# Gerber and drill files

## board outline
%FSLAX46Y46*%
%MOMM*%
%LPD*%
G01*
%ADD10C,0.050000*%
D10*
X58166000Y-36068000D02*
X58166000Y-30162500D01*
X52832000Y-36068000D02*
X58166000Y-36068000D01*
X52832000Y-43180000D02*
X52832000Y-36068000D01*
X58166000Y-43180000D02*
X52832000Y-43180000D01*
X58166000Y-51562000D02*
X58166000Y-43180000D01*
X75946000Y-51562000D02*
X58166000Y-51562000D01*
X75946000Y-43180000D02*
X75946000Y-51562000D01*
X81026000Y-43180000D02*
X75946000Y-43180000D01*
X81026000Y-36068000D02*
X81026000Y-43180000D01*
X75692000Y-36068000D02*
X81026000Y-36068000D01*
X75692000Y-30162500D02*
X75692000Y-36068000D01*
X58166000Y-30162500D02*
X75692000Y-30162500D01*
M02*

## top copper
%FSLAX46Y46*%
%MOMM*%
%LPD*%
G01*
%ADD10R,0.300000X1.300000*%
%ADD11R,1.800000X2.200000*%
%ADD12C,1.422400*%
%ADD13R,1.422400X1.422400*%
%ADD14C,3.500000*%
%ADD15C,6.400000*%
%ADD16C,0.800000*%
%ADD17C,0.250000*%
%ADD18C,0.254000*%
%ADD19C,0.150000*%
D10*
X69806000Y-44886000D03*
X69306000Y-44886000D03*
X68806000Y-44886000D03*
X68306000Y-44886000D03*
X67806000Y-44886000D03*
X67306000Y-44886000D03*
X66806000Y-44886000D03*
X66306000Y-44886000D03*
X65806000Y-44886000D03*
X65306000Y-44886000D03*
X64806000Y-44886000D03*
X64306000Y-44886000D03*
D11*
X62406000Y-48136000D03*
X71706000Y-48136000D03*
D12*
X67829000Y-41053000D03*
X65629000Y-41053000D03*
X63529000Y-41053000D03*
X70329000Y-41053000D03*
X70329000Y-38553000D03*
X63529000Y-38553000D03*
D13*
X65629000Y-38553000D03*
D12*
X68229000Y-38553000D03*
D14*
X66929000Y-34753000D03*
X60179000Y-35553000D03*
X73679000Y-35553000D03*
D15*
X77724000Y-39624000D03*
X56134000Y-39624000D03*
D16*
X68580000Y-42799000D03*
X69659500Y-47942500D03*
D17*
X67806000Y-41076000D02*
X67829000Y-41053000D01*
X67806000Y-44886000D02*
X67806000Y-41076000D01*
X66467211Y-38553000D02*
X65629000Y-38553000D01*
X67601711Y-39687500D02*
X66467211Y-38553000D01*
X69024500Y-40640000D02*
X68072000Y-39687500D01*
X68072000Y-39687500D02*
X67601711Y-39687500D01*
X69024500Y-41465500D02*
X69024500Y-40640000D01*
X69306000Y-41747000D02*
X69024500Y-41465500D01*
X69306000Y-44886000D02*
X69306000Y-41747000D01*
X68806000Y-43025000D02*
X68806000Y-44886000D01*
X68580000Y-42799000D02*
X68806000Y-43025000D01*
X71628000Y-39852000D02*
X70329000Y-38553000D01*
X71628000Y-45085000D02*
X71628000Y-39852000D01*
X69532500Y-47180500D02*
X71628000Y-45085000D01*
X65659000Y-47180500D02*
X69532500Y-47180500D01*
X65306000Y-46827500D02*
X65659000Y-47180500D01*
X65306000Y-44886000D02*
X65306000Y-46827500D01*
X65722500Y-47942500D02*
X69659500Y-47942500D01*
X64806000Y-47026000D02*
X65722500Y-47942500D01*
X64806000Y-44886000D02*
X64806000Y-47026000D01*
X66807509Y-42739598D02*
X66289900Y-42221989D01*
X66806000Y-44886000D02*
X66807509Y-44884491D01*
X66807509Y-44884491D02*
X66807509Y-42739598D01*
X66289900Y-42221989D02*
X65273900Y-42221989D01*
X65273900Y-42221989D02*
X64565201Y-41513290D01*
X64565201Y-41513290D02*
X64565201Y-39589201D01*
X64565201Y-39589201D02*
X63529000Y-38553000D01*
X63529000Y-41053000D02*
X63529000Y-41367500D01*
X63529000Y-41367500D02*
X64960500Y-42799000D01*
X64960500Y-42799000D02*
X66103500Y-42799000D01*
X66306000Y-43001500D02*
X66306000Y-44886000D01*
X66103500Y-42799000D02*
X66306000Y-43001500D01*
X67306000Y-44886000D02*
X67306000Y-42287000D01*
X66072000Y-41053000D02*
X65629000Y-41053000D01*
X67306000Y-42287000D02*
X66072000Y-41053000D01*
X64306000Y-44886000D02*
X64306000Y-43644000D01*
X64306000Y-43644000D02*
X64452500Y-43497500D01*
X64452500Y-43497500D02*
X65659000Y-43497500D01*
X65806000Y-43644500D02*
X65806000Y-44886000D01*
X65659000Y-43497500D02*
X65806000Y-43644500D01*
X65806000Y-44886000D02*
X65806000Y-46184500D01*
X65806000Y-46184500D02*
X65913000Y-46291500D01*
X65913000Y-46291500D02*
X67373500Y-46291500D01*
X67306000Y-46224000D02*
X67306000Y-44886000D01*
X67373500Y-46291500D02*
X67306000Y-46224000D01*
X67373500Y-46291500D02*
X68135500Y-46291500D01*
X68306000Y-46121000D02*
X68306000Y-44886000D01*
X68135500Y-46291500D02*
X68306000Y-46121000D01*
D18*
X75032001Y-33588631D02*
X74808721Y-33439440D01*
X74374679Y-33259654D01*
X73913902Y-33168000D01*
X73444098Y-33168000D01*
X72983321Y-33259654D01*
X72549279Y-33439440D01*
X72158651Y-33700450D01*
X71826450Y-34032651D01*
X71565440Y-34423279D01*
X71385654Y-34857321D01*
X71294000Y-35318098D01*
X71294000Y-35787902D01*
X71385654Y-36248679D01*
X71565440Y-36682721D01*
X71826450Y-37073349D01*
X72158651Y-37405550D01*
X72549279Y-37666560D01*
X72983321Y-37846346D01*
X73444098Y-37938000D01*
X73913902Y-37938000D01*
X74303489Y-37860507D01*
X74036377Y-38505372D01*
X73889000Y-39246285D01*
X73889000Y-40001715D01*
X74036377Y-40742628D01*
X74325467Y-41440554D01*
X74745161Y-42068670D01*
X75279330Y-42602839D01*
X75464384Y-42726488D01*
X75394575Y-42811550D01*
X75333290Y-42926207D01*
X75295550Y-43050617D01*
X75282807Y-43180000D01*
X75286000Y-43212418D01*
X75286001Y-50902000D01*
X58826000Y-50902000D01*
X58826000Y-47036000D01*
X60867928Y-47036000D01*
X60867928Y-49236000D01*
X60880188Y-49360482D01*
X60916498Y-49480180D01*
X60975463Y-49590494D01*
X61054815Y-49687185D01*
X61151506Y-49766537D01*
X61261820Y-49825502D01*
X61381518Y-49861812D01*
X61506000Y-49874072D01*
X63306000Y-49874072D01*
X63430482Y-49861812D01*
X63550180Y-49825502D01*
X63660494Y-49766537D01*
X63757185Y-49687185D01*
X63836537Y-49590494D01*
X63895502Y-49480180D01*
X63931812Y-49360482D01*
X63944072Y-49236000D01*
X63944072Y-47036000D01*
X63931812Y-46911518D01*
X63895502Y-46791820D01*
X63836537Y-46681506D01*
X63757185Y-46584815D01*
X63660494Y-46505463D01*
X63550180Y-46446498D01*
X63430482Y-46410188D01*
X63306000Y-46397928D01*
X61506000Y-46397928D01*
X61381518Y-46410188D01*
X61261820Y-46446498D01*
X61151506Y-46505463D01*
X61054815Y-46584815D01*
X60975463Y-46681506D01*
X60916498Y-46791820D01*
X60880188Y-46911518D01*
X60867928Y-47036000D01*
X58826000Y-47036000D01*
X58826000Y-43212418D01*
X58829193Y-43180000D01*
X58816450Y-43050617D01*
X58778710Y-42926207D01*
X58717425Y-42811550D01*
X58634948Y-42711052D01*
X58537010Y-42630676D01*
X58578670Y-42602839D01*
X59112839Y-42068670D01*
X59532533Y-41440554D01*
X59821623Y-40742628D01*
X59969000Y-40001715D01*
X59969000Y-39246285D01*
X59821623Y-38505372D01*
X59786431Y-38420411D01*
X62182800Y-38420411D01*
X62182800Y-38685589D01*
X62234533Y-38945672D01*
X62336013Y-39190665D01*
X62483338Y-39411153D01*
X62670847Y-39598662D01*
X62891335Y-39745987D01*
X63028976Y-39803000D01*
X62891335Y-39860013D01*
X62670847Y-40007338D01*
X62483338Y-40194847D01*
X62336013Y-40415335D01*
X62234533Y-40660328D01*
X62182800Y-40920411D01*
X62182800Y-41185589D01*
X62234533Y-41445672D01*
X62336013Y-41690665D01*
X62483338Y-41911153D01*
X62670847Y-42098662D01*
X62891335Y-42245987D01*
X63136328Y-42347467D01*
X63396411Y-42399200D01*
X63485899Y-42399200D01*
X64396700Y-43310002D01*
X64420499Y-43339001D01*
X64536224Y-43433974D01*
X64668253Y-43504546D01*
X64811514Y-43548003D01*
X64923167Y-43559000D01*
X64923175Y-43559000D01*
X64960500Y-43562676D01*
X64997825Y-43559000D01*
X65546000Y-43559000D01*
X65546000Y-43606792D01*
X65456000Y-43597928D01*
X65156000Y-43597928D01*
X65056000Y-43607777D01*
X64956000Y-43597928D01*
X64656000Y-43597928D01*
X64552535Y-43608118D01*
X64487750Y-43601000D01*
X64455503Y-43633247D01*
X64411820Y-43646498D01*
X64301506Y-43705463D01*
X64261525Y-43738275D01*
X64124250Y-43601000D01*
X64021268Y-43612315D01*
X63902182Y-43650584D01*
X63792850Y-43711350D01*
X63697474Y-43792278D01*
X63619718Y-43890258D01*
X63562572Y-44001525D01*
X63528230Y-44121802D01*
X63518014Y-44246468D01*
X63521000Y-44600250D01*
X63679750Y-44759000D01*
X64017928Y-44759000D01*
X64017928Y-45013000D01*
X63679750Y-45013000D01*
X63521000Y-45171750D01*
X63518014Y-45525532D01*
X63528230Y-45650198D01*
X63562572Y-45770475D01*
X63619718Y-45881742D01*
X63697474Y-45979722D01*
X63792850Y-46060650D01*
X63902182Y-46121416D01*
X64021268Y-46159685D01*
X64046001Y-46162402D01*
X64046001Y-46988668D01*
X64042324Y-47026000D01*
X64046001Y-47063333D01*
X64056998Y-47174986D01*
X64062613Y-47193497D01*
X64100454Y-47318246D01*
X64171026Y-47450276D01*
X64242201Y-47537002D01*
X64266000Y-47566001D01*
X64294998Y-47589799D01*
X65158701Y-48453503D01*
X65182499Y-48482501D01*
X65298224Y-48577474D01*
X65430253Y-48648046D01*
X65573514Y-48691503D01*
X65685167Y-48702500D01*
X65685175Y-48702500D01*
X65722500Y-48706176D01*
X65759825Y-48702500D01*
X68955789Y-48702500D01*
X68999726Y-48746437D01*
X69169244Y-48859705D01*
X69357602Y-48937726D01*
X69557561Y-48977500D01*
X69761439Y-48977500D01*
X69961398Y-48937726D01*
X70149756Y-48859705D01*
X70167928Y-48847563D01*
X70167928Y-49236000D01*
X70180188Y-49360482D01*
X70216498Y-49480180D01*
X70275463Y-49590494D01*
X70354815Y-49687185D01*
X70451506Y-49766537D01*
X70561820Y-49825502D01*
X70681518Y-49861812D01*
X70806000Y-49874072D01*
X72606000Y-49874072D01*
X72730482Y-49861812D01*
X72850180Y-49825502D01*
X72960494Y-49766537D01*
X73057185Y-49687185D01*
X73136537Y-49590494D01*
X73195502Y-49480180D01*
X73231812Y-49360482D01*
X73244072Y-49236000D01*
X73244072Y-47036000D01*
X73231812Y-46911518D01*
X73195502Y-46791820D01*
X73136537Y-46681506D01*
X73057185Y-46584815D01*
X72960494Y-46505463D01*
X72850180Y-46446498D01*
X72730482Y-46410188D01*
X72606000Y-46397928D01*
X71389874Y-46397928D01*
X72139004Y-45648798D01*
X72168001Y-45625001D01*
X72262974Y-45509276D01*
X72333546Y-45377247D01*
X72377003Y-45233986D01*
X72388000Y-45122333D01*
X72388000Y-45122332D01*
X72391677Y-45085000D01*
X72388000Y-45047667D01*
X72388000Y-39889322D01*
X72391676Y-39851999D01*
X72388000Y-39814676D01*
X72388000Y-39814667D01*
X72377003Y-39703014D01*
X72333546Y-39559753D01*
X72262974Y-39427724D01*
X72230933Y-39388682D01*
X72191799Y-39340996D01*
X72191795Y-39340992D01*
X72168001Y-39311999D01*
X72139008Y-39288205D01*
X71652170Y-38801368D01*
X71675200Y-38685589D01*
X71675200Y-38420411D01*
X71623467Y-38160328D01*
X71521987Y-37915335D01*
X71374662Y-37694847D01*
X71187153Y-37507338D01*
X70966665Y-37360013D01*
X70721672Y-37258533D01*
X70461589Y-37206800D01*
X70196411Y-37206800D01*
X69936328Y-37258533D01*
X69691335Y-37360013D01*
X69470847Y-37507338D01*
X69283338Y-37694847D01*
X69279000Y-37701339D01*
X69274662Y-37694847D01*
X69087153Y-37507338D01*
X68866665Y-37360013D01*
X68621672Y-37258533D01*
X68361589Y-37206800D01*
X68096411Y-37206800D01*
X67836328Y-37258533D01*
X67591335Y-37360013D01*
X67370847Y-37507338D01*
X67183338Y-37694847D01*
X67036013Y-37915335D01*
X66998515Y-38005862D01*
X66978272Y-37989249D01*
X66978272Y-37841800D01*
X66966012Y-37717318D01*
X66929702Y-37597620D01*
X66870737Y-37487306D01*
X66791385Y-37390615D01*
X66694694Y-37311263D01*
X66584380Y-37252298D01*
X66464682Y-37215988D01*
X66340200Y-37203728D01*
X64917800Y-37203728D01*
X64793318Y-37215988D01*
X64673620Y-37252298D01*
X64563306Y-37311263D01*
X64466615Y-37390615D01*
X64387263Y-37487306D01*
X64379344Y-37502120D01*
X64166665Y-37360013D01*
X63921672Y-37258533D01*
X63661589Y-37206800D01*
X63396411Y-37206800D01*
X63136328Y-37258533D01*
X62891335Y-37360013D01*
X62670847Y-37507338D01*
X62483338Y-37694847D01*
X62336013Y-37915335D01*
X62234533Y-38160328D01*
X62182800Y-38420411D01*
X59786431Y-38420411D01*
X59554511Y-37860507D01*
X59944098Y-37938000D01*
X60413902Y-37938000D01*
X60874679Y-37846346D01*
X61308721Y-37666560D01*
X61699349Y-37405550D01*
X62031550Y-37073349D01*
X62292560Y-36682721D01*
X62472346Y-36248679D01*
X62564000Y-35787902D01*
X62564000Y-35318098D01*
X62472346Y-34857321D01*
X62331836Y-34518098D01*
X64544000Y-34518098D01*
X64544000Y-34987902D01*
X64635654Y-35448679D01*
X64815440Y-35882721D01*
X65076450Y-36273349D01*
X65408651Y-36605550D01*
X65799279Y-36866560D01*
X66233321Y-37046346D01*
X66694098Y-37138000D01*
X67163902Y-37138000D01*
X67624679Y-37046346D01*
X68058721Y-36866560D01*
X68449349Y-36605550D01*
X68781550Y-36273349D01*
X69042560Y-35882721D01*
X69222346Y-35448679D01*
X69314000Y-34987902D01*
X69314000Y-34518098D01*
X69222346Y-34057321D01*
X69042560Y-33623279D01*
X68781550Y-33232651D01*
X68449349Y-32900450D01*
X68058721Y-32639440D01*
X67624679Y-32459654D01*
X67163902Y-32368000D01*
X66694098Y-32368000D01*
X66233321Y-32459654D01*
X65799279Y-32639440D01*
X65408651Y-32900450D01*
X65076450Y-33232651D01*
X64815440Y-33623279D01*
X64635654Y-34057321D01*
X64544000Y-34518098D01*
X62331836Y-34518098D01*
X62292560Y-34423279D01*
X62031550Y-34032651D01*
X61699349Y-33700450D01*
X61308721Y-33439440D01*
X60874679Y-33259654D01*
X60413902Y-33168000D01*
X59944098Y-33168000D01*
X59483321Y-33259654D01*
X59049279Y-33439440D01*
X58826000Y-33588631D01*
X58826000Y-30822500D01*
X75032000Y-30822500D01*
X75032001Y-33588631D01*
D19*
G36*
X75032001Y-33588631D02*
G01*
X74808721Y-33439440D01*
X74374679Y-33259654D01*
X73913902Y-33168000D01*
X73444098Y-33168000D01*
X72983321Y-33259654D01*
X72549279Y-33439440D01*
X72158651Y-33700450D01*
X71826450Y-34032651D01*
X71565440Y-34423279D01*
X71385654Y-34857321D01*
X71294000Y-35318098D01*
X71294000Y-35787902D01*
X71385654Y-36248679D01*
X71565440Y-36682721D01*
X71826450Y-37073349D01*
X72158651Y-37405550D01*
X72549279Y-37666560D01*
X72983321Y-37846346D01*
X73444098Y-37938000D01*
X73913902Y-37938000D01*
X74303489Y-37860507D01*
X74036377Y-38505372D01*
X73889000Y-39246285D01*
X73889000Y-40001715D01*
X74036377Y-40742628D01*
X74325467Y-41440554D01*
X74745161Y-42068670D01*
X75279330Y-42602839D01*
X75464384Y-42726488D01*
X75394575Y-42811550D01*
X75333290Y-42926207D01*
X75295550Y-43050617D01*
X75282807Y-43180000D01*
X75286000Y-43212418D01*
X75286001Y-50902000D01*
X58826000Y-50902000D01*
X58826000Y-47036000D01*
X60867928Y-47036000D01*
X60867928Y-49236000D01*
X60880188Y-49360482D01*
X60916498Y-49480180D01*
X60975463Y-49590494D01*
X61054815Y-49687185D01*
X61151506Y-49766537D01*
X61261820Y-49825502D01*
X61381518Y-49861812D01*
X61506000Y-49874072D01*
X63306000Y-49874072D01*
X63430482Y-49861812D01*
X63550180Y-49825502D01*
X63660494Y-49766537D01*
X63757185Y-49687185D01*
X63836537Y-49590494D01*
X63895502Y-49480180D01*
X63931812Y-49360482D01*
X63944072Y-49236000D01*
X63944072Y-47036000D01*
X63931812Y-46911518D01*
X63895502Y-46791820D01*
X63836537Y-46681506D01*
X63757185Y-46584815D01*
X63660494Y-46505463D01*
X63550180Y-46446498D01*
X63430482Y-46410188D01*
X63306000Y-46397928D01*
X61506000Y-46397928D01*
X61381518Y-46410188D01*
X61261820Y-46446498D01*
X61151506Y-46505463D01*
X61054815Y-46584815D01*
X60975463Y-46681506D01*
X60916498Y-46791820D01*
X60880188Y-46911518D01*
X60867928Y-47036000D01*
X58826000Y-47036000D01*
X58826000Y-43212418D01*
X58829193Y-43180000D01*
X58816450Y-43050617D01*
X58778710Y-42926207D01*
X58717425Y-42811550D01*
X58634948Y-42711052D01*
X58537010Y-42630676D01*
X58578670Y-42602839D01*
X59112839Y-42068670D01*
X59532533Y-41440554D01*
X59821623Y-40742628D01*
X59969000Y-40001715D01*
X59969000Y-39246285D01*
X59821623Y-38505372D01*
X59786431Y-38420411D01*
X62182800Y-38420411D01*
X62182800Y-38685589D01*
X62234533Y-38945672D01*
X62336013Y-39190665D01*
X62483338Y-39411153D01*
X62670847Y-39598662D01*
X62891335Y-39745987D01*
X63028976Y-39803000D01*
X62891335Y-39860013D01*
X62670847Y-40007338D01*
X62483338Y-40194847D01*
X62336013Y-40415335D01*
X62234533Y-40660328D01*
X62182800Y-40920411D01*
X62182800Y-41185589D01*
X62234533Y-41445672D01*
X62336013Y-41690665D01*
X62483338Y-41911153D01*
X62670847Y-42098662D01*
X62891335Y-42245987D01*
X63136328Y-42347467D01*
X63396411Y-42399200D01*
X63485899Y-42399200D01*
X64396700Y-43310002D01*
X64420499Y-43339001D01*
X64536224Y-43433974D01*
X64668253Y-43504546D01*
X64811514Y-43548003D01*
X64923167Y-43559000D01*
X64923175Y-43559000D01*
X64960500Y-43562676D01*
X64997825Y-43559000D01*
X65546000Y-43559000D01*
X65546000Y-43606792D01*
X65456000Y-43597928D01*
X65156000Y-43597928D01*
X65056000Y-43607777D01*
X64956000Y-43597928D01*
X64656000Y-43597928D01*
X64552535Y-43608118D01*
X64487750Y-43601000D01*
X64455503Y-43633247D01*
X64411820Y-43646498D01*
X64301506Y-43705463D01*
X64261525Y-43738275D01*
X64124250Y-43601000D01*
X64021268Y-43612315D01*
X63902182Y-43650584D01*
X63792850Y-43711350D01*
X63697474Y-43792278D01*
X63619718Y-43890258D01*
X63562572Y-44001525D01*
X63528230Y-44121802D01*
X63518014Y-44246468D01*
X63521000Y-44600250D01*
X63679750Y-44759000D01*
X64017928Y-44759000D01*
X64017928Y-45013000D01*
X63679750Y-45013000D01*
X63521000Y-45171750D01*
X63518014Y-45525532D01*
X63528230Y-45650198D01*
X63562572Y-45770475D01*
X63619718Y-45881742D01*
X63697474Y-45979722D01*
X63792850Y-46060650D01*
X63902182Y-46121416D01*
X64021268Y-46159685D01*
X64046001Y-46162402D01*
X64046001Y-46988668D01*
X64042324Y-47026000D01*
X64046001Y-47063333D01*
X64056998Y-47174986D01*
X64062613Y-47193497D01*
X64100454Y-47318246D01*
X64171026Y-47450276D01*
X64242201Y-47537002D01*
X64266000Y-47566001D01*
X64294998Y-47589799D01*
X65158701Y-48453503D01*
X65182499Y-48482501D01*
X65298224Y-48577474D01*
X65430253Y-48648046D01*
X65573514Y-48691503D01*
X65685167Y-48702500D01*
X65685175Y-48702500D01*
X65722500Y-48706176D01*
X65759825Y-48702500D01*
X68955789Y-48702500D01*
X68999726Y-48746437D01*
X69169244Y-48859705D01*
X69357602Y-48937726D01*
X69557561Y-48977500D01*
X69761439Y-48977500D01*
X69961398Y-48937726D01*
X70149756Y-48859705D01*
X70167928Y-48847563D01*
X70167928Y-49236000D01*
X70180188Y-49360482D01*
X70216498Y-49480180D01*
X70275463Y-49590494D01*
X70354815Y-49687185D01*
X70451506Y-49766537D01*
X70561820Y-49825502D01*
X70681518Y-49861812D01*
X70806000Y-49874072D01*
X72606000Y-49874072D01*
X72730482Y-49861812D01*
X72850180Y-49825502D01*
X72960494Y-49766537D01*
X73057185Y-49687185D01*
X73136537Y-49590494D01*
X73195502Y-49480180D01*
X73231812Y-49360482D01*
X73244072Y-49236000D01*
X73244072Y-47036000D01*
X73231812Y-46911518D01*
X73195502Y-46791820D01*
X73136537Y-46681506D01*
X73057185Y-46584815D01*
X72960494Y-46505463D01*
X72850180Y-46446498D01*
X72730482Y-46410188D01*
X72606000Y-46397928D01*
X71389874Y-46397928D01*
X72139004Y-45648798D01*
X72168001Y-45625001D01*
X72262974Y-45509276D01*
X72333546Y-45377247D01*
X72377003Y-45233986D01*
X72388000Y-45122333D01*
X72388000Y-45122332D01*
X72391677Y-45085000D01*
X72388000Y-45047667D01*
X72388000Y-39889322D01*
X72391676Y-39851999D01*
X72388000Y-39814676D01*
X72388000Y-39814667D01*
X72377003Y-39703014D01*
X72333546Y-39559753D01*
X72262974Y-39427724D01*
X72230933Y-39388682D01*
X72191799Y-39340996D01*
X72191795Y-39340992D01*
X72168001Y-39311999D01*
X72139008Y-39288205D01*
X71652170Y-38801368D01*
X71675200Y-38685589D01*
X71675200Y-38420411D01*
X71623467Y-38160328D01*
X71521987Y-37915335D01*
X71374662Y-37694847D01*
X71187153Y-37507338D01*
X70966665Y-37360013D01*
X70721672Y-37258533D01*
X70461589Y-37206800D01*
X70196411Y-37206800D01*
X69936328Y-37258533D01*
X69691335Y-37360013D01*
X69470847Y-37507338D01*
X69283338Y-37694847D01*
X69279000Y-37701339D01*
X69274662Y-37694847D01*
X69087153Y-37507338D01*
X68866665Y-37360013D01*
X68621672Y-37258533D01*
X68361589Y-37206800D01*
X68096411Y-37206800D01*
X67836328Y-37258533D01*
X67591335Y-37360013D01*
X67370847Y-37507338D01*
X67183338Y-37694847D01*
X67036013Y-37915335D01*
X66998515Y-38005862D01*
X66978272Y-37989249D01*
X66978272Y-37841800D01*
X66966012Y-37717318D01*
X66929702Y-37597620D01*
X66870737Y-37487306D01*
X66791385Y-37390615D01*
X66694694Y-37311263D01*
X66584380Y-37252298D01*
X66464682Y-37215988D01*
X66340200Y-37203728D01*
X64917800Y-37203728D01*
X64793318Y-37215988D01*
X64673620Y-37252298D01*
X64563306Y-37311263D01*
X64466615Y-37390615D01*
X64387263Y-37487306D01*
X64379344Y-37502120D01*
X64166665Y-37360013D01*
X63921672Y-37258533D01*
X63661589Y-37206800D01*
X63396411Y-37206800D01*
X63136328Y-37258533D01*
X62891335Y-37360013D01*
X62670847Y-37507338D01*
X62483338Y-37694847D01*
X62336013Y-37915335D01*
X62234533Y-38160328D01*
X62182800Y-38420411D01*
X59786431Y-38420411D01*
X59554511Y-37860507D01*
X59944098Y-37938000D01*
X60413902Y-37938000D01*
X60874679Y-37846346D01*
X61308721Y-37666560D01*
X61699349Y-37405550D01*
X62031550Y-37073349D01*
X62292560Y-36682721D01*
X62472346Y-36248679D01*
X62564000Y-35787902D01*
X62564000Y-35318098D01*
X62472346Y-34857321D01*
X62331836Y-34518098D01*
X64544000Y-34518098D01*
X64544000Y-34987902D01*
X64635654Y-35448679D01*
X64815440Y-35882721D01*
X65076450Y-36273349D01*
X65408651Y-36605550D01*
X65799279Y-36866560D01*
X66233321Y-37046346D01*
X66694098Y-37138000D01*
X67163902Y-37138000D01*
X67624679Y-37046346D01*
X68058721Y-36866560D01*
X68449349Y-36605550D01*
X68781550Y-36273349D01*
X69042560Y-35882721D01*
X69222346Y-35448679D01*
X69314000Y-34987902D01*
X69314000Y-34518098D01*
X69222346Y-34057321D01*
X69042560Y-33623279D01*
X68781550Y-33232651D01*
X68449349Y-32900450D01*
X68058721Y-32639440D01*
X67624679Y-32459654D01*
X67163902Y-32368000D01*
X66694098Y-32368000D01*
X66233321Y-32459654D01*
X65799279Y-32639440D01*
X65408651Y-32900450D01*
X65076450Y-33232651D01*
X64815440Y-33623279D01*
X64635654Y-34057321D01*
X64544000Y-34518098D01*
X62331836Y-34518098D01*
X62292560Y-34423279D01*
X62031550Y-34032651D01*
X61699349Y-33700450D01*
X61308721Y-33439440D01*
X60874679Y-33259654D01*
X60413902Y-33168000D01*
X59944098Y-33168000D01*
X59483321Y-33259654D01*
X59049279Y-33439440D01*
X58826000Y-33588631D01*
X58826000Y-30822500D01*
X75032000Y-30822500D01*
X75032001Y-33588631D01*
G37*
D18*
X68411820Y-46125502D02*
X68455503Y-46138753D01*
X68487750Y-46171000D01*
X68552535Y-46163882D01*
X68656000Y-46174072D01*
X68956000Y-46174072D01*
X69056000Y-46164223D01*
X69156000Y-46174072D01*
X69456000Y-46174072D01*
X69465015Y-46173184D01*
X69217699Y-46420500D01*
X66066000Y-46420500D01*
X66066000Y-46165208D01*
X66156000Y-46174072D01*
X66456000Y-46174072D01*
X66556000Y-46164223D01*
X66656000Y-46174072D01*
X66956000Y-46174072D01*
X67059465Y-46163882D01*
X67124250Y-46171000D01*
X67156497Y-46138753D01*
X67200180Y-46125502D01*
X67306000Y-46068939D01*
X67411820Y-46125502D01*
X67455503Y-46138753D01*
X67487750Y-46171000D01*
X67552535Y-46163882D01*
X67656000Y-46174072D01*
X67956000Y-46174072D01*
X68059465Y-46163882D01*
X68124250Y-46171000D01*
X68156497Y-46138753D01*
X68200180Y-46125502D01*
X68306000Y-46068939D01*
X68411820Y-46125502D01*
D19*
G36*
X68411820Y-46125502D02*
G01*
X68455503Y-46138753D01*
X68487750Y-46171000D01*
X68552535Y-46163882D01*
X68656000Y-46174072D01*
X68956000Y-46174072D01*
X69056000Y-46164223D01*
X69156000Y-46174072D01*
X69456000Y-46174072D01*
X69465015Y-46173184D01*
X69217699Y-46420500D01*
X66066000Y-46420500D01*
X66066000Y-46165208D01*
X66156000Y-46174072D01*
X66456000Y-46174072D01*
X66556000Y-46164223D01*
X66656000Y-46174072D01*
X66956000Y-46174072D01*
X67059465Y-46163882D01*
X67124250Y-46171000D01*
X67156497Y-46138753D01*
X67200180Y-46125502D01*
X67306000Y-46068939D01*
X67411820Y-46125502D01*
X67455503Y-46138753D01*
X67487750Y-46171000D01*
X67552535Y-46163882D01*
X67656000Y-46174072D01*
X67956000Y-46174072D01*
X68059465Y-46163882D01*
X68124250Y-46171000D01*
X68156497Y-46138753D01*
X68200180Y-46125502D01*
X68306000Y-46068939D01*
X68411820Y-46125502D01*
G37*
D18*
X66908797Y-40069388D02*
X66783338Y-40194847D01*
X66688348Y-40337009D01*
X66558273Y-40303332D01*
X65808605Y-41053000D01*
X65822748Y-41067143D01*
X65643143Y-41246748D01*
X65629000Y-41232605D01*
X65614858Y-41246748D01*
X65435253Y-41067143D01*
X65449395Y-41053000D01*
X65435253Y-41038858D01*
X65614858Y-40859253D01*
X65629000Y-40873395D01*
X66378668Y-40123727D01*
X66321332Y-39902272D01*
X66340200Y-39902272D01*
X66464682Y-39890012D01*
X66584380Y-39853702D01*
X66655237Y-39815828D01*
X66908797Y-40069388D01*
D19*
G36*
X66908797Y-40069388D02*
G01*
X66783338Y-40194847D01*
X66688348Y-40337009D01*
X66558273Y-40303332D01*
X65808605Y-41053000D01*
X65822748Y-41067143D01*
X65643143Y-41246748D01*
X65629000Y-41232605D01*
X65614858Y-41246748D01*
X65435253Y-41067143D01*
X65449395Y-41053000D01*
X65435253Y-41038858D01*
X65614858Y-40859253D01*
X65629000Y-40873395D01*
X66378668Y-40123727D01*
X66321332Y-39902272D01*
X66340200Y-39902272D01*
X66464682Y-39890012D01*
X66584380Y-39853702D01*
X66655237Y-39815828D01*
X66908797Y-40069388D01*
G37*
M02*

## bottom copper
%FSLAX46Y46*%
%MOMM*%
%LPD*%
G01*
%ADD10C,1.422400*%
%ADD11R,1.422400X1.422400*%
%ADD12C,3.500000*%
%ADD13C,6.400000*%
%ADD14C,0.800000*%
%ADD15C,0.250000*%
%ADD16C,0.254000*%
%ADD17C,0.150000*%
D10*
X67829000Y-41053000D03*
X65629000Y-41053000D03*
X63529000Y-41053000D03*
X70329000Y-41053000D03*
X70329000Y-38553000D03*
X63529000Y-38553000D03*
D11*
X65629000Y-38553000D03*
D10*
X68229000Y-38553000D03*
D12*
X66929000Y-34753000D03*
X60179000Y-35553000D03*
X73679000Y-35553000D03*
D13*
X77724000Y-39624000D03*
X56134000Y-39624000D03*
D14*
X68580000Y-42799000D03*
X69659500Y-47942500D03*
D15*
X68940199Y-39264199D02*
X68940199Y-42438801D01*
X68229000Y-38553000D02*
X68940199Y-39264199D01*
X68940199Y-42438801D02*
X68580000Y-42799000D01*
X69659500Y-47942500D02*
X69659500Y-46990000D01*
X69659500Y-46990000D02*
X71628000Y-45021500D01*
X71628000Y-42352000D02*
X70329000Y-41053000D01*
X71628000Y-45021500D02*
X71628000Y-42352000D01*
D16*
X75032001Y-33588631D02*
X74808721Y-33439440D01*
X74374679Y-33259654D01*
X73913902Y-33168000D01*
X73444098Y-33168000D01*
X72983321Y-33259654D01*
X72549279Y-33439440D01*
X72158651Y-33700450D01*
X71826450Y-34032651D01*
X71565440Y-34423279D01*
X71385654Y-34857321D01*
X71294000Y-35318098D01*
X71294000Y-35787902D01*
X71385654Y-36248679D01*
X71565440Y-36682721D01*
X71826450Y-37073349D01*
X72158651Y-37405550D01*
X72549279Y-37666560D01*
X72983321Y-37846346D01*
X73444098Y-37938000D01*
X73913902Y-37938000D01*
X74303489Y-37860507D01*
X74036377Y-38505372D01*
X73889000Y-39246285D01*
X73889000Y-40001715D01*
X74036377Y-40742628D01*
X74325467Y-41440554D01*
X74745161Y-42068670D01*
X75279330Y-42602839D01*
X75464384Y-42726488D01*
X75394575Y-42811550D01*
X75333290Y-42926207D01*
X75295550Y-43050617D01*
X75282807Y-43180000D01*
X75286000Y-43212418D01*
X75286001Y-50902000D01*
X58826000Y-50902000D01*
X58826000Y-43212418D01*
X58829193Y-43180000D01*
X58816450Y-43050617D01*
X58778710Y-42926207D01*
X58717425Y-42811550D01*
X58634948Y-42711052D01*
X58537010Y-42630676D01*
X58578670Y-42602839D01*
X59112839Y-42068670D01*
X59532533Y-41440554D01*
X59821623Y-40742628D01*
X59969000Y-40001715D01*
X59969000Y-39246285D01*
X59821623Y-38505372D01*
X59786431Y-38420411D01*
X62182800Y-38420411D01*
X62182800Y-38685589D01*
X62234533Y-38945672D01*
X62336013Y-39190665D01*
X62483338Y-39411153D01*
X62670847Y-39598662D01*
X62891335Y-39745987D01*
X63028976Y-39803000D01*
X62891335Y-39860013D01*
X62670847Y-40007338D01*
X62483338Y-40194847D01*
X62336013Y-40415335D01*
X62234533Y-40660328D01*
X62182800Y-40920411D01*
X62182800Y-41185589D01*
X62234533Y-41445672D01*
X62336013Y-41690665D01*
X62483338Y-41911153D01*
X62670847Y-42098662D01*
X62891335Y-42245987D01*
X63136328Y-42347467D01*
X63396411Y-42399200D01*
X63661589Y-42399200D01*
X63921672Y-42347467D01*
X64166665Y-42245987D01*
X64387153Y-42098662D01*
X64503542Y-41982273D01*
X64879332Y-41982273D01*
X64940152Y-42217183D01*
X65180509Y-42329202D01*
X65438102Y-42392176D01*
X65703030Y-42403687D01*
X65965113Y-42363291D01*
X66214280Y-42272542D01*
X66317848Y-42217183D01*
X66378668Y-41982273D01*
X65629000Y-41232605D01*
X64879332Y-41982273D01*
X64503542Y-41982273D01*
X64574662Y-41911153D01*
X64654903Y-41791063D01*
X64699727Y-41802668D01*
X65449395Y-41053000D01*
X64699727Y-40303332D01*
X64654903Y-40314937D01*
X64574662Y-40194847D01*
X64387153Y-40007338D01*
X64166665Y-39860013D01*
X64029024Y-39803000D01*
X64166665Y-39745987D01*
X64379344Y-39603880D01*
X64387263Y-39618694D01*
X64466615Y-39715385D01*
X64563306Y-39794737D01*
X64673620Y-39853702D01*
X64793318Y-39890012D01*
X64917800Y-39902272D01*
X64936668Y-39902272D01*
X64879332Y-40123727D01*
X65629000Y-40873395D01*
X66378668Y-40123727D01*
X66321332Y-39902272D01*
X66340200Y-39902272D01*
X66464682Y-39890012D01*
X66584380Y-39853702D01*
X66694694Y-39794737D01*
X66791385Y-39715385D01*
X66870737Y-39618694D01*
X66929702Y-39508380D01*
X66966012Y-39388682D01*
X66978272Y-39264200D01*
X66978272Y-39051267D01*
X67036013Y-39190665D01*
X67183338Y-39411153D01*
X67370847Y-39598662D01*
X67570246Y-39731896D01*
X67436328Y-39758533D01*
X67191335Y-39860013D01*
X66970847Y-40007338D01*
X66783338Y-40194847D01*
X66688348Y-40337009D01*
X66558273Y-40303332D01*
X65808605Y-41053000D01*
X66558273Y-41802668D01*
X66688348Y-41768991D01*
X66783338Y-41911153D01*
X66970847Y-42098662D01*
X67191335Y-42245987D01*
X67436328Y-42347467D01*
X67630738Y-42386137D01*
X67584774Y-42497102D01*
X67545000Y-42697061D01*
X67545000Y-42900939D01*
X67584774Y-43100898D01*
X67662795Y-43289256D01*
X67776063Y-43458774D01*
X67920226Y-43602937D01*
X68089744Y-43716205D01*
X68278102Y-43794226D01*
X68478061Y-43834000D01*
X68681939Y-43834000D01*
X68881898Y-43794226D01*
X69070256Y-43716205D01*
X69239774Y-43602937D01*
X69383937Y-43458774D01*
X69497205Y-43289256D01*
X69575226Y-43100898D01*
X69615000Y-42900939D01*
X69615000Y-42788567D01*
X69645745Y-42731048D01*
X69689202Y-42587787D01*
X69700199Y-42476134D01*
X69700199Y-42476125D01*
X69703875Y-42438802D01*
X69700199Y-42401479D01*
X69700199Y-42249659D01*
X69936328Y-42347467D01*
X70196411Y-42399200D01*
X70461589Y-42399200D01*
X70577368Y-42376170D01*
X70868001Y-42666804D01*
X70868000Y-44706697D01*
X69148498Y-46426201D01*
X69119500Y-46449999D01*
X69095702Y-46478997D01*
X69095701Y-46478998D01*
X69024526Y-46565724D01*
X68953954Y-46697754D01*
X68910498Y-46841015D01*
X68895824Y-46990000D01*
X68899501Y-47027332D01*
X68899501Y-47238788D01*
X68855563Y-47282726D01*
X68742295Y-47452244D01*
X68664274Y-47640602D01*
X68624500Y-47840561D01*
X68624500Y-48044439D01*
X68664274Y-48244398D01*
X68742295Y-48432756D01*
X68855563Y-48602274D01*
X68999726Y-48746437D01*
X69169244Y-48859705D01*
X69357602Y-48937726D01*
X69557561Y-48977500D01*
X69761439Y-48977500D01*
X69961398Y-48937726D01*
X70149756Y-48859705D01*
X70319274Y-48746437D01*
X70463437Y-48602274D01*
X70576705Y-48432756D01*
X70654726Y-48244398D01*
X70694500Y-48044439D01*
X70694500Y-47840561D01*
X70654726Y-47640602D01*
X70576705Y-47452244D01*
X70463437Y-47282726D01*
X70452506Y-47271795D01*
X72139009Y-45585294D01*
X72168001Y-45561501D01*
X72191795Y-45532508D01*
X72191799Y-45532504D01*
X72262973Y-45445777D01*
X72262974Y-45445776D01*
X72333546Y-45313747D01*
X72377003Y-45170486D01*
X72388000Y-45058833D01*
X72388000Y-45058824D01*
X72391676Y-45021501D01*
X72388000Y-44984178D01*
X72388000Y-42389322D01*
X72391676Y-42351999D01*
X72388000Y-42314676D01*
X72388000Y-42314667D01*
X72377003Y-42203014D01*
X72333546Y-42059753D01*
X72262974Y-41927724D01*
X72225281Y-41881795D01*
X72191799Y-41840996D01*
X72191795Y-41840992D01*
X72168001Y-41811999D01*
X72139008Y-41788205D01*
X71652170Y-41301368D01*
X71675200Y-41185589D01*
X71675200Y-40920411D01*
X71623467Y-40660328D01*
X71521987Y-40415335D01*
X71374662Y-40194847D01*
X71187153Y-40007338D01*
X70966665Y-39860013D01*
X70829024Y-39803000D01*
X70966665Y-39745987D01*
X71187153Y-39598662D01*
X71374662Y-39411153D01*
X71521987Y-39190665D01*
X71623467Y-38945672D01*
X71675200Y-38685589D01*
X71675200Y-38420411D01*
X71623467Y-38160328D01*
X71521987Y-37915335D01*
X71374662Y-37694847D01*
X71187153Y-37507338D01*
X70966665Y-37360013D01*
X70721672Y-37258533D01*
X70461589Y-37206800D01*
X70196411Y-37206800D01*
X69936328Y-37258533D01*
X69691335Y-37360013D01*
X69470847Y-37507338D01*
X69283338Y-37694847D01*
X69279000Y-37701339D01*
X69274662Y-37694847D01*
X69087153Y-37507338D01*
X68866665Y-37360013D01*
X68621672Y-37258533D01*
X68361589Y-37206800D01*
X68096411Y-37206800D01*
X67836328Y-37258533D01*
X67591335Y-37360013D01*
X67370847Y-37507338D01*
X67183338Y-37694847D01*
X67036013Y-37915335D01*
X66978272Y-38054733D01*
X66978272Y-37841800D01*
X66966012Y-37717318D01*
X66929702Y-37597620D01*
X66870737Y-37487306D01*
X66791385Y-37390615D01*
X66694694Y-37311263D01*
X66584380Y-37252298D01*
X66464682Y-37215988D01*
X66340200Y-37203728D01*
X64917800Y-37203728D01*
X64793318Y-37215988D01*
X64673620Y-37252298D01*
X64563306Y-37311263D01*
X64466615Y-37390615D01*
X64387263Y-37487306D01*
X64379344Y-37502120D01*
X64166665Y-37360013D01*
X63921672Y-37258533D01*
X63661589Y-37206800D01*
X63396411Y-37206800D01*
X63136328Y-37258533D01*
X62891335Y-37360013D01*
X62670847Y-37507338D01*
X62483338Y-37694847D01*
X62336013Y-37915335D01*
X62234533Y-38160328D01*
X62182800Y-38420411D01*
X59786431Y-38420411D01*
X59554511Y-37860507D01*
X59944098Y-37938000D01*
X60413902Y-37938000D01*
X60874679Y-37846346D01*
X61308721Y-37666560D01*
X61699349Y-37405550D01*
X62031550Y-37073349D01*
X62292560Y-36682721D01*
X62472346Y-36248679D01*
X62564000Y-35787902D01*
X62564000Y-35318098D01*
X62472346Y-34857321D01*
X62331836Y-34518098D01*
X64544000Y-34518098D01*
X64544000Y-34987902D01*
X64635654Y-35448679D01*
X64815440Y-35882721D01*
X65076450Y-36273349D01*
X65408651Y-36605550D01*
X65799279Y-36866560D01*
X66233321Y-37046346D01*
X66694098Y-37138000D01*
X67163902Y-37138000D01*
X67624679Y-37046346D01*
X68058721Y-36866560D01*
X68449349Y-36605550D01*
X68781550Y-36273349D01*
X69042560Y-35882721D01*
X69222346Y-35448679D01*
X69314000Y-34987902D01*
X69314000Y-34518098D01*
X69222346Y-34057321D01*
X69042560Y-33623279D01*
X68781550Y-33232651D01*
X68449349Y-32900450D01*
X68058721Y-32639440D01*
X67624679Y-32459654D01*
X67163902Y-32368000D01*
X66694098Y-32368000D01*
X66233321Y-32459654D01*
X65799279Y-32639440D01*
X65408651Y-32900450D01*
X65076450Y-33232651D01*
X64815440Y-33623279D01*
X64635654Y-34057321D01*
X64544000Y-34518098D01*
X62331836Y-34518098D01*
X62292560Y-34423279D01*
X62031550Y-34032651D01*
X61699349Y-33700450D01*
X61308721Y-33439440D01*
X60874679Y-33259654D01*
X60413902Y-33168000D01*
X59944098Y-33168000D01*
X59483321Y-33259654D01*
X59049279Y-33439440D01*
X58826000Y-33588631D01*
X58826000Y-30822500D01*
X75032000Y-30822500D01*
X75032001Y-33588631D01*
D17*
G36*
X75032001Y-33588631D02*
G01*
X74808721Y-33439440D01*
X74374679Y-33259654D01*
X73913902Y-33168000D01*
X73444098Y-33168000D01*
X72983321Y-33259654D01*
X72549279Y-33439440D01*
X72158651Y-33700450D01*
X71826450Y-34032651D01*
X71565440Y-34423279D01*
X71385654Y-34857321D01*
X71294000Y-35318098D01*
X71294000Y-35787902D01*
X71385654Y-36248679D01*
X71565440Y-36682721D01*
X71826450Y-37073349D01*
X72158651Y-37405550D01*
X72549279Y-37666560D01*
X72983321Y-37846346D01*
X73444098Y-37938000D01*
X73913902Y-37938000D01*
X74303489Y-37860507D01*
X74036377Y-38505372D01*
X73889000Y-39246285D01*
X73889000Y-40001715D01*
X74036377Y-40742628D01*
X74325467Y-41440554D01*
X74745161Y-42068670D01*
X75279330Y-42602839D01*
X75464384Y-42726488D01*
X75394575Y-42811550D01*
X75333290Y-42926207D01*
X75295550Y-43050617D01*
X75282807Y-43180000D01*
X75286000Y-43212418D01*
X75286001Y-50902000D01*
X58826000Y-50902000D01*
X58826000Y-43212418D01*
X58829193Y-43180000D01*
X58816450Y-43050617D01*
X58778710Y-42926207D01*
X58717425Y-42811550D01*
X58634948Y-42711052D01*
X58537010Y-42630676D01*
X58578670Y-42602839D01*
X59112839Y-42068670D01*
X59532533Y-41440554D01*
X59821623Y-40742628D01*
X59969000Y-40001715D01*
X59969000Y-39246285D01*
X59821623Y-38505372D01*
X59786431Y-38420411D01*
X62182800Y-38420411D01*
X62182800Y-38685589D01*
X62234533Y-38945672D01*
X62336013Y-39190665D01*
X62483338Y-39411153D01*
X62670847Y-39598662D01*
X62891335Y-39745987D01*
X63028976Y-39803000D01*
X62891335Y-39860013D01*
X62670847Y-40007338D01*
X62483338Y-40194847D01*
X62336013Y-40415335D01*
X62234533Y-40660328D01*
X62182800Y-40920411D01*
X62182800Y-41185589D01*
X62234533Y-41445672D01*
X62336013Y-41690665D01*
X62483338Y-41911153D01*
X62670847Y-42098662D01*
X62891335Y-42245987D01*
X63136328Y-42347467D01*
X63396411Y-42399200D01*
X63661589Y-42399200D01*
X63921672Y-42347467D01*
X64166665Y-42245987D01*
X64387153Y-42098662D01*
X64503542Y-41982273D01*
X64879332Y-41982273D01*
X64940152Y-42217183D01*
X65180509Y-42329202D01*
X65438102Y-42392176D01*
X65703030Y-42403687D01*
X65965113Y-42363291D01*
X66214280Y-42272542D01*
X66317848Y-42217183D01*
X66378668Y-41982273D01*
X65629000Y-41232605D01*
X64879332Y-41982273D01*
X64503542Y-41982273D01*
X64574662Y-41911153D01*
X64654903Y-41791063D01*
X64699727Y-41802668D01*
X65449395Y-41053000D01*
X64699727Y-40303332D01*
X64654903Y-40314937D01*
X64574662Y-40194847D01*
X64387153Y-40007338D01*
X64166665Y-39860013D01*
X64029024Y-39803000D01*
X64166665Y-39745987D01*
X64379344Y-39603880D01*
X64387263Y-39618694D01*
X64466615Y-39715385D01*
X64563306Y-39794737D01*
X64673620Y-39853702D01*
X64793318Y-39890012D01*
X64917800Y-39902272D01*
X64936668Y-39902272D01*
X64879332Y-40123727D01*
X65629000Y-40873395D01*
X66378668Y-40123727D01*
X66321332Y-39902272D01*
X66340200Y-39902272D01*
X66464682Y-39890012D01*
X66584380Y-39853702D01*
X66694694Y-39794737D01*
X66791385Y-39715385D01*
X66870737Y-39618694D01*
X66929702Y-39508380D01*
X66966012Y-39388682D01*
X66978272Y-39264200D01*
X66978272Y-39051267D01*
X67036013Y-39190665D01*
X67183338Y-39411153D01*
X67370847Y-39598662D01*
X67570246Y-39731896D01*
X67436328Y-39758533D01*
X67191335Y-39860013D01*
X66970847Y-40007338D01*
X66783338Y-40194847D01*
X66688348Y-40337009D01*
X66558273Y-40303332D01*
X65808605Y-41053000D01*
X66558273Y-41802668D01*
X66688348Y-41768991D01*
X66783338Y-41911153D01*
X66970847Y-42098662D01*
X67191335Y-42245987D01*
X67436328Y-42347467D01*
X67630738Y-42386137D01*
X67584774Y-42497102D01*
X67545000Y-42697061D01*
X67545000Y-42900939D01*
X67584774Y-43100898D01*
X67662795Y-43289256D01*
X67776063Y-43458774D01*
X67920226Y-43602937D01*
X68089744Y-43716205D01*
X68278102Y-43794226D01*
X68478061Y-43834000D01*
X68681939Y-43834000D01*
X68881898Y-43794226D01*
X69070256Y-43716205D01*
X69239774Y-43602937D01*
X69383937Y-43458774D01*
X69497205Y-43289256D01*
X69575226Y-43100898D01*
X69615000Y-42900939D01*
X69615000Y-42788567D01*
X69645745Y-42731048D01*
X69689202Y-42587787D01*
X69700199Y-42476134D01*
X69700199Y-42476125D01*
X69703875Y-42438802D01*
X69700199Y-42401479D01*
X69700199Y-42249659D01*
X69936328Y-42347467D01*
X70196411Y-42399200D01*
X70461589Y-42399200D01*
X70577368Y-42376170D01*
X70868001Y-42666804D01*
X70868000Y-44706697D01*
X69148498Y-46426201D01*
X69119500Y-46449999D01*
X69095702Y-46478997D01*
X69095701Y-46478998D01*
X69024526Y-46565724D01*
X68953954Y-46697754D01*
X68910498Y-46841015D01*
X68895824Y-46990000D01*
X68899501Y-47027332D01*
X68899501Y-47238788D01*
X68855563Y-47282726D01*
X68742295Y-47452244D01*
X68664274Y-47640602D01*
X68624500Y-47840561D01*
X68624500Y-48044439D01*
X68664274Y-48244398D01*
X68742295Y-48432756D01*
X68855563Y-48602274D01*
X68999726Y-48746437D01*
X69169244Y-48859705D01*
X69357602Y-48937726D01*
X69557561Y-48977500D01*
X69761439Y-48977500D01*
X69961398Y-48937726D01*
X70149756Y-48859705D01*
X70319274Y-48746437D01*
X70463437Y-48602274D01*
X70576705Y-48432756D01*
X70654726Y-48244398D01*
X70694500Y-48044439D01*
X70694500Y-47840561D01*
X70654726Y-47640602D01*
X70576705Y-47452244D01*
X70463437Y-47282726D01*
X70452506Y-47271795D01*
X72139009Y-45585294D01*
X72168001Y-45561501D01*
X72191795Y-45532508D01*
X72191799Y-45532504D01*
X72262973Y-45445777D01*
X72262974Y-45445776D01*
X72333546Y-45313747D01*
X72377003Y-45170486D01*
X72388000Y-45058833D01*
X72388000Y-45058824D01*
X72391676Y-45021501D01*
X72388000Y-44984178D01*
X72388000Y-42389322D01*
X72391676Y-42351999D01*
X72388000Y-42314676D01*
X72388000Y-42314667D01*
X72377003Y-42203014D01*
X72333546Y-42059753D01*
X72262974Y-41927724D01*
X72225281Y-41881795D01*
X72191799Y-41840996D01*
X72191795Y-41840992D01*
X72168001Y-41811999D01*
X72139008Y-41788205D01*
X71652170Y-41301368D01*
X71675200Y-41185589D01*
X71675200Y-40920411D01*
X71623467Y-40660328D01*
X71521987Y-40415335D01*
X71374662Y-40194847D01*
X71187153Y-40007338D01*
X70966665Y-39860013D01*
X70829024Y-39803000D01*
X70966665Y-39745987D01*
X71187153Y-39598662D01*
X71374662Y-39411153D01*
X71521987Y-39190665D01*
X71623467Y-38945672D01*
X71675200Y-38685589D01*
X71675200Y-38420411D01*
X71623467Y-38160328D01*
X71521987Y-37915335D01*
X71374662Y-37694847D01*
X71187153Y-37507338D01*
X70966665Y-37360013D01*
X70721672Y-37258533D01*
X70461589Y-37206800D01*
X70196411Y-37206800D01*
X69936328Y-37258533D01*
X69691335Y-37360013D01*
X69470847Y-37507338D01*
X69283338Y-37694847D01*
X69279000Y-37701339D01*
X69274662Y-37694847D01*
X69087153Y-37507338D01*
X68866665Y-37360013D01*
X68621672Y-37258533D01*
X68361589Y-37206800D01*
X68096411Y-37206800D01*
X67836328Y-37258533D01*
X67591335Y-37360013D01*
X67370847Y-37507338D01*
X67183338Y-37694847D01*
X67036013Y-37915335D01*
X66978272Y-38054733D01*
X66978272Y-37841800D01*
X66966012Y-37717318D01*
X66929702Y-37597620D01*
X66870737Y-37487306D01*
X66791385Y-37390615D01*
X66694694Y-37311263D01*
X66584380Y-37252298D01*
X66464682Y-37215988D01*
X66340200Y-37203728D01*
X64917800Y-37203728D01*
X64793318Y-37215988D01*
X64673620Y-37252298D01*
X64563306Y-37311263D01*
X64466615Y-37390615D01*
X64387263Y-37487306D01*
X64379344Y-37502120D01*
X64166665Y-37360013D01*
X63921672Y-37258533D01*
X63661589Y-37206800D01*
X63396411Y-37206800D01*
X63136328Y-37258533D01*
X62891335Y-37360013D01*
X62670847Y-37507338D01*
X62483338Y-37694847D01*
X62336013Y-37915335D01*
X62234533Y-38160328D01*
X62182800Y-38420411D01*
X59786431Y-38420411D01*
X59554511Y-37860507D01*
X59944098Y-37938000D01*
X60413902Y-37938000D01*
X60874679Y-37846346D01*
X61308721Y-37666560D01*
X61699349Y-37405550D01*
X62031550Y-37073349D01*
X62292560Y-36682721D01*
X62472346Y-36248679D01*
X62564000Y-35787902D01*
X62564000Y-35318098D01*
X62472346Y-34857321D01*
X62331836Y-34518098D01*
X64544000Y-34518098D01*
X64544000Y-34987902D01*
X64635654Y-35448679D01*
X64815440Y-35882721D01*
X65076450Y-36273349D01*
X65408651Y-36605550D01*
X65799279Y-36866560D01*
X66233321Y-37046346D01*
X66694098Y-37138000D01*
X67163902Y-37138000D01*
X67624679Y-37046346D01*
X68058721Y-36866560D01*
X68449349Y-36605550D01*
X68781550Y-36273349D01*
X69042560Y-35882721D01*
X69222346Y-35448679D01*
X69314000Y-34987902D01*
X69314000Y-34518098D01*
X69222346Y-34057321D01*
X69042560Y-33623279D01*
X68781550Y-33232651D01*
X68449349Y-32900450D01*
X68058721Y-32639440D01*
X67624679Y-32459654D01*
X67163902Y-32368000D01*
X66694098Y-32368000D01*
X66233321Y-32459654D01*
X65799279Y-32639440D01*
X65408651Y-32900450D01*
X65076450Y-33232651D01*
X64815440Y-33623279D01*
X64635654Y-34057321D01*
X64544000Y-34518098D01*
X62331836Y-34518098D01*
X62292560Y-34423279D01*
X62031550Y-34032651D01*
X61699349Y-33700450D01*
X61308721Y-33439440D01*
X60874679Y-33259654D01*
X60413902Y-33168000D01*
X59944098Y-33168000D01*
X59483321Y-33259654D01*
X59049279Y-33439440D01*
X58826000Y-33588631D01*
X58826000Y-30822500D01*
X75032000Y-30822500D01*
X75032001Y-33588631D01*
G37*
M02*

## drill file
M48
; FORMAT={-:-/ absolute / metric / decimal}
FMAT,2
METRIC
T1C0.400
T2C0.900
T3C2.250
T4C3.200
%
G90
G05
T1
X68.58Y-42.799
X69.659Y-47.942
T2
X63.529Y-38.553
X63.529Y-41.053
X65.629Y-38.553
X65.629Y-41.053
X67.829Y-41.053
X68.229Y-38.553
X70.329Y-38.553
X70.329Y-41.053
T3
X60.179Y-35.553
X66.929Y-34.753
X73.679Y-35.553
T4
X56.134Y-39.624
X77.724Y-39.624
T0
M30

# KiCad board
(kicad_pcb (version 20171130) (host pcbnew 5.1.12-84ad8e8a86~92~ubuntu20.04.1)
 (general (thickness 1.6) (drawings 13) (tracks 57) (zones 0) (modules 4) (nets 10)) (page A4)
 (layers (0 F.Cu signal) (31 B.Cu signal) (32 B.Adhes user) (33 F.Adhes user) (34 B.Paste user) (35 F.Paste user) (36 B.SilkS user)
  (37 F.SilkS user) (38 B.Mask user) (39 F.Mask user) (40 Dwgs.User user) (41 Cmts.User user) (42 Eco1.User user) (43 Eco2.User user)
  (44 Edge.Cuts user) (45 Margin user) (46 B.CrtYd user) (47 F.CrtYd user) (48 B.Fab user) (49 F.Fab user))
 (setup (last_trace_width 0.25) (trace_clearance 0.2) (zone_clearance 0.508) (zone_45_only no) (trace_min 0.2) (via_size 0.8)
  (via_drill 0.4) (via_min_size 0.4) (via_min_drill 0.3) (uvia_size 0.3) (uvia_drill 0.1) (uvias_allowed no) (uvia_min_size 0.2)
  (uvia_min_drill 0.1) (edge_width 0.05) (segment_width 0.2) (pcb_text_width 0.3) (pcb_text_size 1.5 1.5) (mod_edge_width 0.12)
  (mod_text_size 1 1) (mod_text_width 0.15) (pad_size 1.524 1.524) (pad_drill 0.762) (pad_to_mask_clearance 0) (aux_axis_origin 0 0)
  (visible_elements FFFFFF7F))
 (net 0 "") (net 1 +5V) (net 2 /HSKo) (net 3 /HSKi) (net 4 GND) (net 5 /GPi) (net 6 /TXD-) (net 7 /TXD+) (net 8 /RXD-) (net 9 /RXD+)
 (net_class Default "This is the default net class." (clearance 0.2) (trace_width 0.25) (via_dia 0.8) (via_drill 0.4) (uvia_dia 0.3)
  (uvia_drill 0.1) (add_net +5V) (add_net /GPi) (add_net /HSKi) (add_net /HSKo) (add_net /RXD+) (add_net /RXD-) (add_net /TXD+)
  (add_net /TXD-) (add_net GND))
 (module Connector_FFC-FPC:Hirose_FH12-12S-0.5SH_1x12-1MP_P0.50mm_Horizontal (layer F.Cu) (at 67.056 46.736)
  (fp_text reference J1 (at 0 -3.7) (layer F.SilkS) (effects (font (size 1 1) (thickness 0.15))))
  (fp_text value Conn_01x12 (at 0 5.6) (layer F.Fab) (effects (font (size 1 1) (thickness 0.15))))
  (pad 12 smd rect (at 2.75 -1.85) (size 0.3 1.3) (layers F.Cu F.Paste F.Mask) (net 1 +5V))
  (pad 11 smd rect (at 2.25 -1.85) (size 0.3 1.3) (layers F.Cu F.Paste F.Mask) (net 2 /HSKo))
  (pad 10 smd rect (at 1.75 -1.85) (size 0.3 1.3) (layers F.Cu F.Paste F.Mask) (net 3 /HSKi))
  (pad 9 smd rect (at 1.25 -1.85) (size 0.3 1.3) (layers F.Cu F.Paste F.Mask) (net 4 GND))
  (pad 8 smd rect (at 0.75 -1.85) (size 0.3 1.3) (layers F.Cu F.Paste F.Mask) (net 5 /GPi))
  (pad 7 smd rect (at 0.25 -1.85) (size 0.3 1.3) (layers F.Cu F.Paste F.Mask) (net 4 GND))
  (pad 6 smd rect (at -0.25 -1.85) (size 0.3 1.3) (layers F.Cu F.Paste F.Mask) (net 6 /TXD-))
  (pad 5 smd rect (at -0.75 -1.85) (size 0.3 1.3) (layers F.Cu F.Paste F.Mask) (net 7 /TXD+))
  (pad 4 smd rect (at -1.25 -1.85) (size 0.3 1.3) (layers F.Cu F.Paste F.Mask) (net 4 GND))
  (pad 3 smd rect (at -1.75 -1.85) (size 0.3 1.3) (layers F.Cu F.Paste F.Mask) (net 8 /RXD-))
  (pad 2 smd rect (at -2.25 -1.85) (size 0.3 1.3) (layers F.Cu F.Paste F.Mask) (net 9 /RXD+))
  (pad 1 smd rect (at -2.75 -1.85) (size 0.3 1.3) (layers F.Cu F.Paste F.Mask) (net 4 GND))
  (pad MP smd rect (at -4.65 1.4) (size 1.8 2.2) (layers F.Cu F.Paste F.Mask))
  (pad MP smd rect (at 4.65 1.4) (size 1.8 2.2) (layers F.Cu F.Paste F.Mask)))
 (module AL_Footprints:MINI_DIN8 (layer F.Cu) (at 66.929 34.753)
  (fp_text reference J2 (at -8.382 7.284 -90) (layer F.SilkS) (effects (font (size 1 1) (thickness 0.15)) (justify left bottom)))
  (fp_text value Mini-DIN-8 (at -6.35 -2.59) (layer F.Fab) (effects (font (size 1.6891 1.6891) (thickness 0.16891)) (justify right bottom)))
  (pad 7 thru_hole circle (at 0.9 6.3) (size 1.4224 1.4224) (drill 0.9) (layers *.Cu *.Mask) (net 5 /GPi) (solder_mask_margin 0.0508))
  (pad 4 thru_hole circle (at -1.3 6.3) (size 1.4224 1.4224) (drill 0.9) (layers *.Cu *.Mask) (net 4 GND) (solder_mask_margin 0.0508))
  (pad 6 thru_hole circle (at -3.4 6.3) (size 1.4224 1.4224) (drill 0.9) (layers *.Cu *.Mask) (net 7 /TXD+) (solder_mask_margin 0.0508))
  (pad 8 thru_hole circle (at 3.4 6.3) (size 1.4224 1.4224) (drill 0.9) (layers *.Cu *.Mask) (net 9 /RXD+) (solder_mask_margin 0.0508))
  (pad 5 thru_hole circle (at 3.4 3.8) (size 1.4224 1.4224) (drill 0.9) (layers *.Cu *.Mask) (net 8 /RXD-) (solder_mask_margin 0.0508))
  (pad 3 thru_hole circle (at -3.4 3.8) (size 1.4224 1.4224) (drill 0.9) (layers *.Cu *.Mask) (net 6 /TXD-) (solder_mask_margin 0.0508))
  (pad 1 thru_hole rect (at -1.3 3.8) (size 1.4224 1.4224) (drill 0.9) (layers *.Cu *.Mask) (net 2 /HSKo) (solder_mask_margin 0.0508))
  (pad 2 thru_hole circle (at 1.3 3.8) (size 1.4224 1.4224) (drill 0.9) (layers *.Cu *.Mask) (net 3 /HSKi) (solder_mask_margin 0.0508))
  (pad SH2 thru_hole circle (at 0 0) (size 3.5 3.5) (drill 2.25) (layers *.Cu *.Mask) (solder_mask_margin 0.0508))
  (pad SH3 thru_hole circle (at -6.75 0.8) (size 3.5 3.5) (drill 2.25) (layers *.Cu *.Mask) (solder_mask_margin 0.0508))
  (pad SH1 thru_hole circle (at 6.75 0.8) (size 3.5 3.5) (drill 2.25) (layers *.Cu *.Mask) (solder_mask_margin 0.0508)))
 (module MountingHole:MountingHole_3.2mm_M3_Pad (layer F.Cu) (at 77.724 39.624)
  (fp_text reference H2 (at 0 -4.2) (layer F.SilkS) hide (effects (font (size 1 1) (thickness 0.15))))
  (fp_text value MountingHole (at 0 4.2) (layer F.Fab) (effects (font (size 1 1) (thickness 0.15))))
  (pad 1 thru_hole circle (at 0 0) (size 6.4 6.4) (drill 3.2) (layers *.Cu *.Mask)))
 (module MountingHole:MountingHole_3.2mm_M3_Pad (layer F.Cu) (at 56.134 39.624)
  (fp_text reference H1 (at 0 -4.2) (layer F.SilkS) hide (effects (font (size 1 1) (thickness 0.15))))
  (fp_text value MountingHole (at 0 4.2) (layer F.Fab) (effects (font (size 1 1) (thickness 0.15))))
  (pad 1 thru_hole circle (at 0 0) (size 6.4 6.4) (drill 3.2) (layers *.Cu *.Mask)))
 (gr_line (start 58.166 36.068) (end 58.166 30.1625) (layer Edge.Cuts) (width 0.05))
 (gr_line (start 52.832 36.068) (end 58.166 36.068) (layer Edge.Cuts) (width 0.05))
 (gr_line (start 52.832 43.18) (end 52.832 36.068) (layer Edge.Cuts) (width 0.05))
 (gr_line (start 58.166 43.18) (end 52.832 43.18) (layer Edge.Cuts) (width 0.05))
 (gr_line (start 58.166 51.562) (end 58.166 43.18) (layer Edge.Cuts) (width 0.05))
 (gr_line (start 75.946 51.562) (end 58.166 51.562) (layer Edge.Cuts) (width 0.05))
 (gr_line (start 75.946 43.18) (end 75.946 51.562) (layer Edge.Cuts) (width 0.05))
 (gr_line (start 81.026 43.18) (end 75.946 43.18) (layer Edge.Cuts) (width 0.05))
 (gr_line (start 81.026 36.068) (end 81.026 43.18) (layer Edge.Cuts) (width 0.05))
 (gr_line (start 75.692 36.068) (end 81.026 36.068) (layer Edge.Cuts) (width 0.05))
 (gr_line (start 75.692 30.1625) (end 75.692 36.068) (layer Edge.Cuts) (width 0.05))
 (gr_line (start 58.166 30.1625) (end 75.692 30.1625) (layer Edge.Cuts) (width 0.05))
 (segment (start 67.806 41.076) (end 67.829 41.053) (width 0.25) (layer F.Cu) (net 5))
 (segment (start 67.806 44.886) (end 67.806 41.076) (width 0.25) (layer F.Cu) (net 5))
 (segment (start 66.467211 38.553) (end 65.629 38.553) (width 0.25) (layer F.Cu) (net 2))
 (segment (start 67.601711 39.6875) (end 66.467211 38.553) (width 0.25) (layer F.Cu) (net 2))
 (segment (start 69.0245 40.64) (end 68.072 39.6875) (width 0.25) (layer F.Cu) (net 2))
 (segment (start 68.072 39.6875) (end 67.601711 39.6875) (width 0.25) (layer F.Cu) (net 2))
 (segment (start 69.0245 41.4655) (end 69.0245 40.64) (width 0.25) (layer F.Cu) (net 2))
 (segment (start 69.306 41.747) (end 69.0245 41.4655) (width 0.25) (layer F.Cu) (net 2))
 (segment (start 69.306 44.886) (end 69.306 41.747) (width 0.25) (layer F.Cu) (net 2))
 (via (at 68.58 42.799) (size 0.8) (drill 0.4) (layers F.Cu B.Cu) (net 3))
 (segment (start 68.940199 39.264199) (end 68.940199 42.438801) (width 0.25) (layer B.Cu) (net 3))
 (segment (start 68.229 38.553) (end 68.940199 39.264199) (width 0.25) (layer B.Cu) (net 3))
 (segment (start 68.940199 42.438801) (end 68.58 42.799) (width 0.25) (layer B.Cu) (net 3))
 (segment (start 68.806 43.025) (end 68.806 44.886) (width 0.25) (layer F.Cu) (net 3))
 (segment (start 68.58 42.799) (end 68.806 43.025) (width 0.25) (layer F.Cu) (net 3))
 (segment (start 71.628 39.852) (end 70.329 38.553) (width 0.25) (layer F.Cu) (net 8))
 (segment (start 71.628 45.085) (end 71.628 39.852) (width 0.25) (layer F.Cu) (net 8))
 (segment (start 69.5325 47.1805) (end 71.628 45.085) (width 0.25) (layer F.Cu) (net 8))
 (segment (start 65.659 47.1805) (end 69.5325 47.1805) (width 0.25) (layer F.Cu) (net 8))
 (segment (start 65.306 46.8275) (end 65.659 47.1805) (width 0.25) (layer F.Cu) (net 8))
 (segment (start 65.306 44.886) (end 65.306 46.8275) (width 0.25) (layer F.Cu) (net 8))
 (via (at 69.6595 47.9425) (size 0.8) (drill 0.4) (layers F.Cu B.Cu) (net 9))
 (segment (start 69.6595 47.9425) (end 69.6595 46.99) (width 0.25) (layer B.Cu) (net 9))
 (segment (start 69.6595 46.99) (end 71.628 45.0215) (width 0.25) (layer B.Cu) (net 9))
 (segment (start 71.628 42.352) (end 70.329 41.053) (width 0.25) (layer B.Cu) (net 9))
 (segment (start 71.628 45.0215) (end 71.628 42.352) (width 0.25) (layer B.Cu) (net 9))
 (segment (start 65.7225 47.9425) (end 69.6595 47.9425) (width 0.25) (layer F.Cu) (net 9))
 (segment (start 64.806 47.026) (end 65.7225 47.9425) (width 0.25) (layer F.Cu) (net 9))
 (segment (start 64.806 44.886) (end 64.806 47.026) (width 0.25) (layer F.Cu) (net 9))
 (segment (start 66.807509 42.739598) (end 66.2899 42.221989) (width 0.25) (layer F.Cu) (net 6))
 (segment (start 66.806 44.886) (end 66.807509 44.884491) (width 0.25) (layer F.Cu) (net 6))
 (segment (start 66.807509 44.884491) (end 66.807509 42.739598) (width 0.25) (layer F.Cu) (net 6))
 (segment (start 66.2899 42.221989) (end 65.2739 42.221989) (width 0.25) (layer F.Cu) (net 6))
 (segment (start 65.2739 42.221989) (end 64.565201 41.51329) (width 0.25) (layer F.Cu) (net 6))
 (segment (start 64.565201 41.51329) (end 64.565201 39.589201) (width 0.25) (layer F.Cu) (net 6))
 (segment (start 64.565201 39.589201) (end 63.529 38.553) (width 0.25) (layer F.Cu) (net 6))
 (segment (start 63.529 41.053) (end 63.529 41.3675) (width 0.25) (layer F.Cu) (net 7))
 (segment (start 63.529 41.3675) (end 64.9605 42.799) (width 0.25) (layer F.Cu) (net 7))
 (segment (start 64.9605 42.799) (end 66.1035 42.799) (width 0.25) (layer F.Cu) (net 7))
 (segment (start 66.306 43.0015) (end 66.306 44.886) (width 0.25) (layer F.Cu) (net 7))
 (segment (start 66.1035 42.799) (end 66.306 43.0015) (width 0.25) (layer F.Cu) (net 7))
 (segment (start 67.306 44.886) (end 67.306 42.287) (width 0.25) (layer F.Cu) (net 4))
 (segment (start 66.072 41.053) (end 65.629 41.053) (width 0.25) (layer F.Cu) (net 4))
 (segment (start 67.306 42.287) (end 66.072 41.053) (width 0.25) (layer F.Cu) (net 4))
 (segment (start 64.306 44.886) (end 64.306 43.644) (width 0.25) (layer F.Cu) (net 4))
 (segment (start 64.306 43.644) (end 64.4525 43.4975) (width 0.25) (layer F.Cu) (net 4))
 (segment (start 64.4525 43.4975) (end 65.659 43.4975) (width 0.25) (layer F.Cu) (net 4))
 (segment (start 65.806 43.6445) (end 65.806 44.886) (width 0.25) (layer F.Cu) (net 4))
 (segment (start 65.659 43.4975) (end 65.806 43.6445) (width 0.25) (layer F.Cu) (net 4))
 (segment (start 65.806 44.886) (end 65.806 46.1845) (width 0.25) (layer F.Cu) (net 4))
 (segment (start 65.806 46.1845) (end 65.913 46.2915) (width 0.25) (layer F.Cu) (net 4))
 (segment (start 65.913 46.2915) (end 67.3735 46.2915) (width 0.25) (layer F.Cu) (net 4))
 (segment (start 67.306 46.224) (end 67.306 44.886) (width 0.25) (layer F.Cu) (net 4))
 (segment (start 67.3735 46.2915) (end 67.306 46.224) (width 0.25) (layer F.Cu) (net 4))
 (segment (start 67.3735 46.2915) (end 68.1355 46.2915) (width 0.25) (layer F.Cu) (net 4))
 (segment (start 68.306 46.121) (end 68.306 44.886) (width 0.25) (layer F.Cu) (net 4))
 (segment (start 68.1355 46.2915) (end 68.306 46.121) (width 0.25) (layer F.Cu) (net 4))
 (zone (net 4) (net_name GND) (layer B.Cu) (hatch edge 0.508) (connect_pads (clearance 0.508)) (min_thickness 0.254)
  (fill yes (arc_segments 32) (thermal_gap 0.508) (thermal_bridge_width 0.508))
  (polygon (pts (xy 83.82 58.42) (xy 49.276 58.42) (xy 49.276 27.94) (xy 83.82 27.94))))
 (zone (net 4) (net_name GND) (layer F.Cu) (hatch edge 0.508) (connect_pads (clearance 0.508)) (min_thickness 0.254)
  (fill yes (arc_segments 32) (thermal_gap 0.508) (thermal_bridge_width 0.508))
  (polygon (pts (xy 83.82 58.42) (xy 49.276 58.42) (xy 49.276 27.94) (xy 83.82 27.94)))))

